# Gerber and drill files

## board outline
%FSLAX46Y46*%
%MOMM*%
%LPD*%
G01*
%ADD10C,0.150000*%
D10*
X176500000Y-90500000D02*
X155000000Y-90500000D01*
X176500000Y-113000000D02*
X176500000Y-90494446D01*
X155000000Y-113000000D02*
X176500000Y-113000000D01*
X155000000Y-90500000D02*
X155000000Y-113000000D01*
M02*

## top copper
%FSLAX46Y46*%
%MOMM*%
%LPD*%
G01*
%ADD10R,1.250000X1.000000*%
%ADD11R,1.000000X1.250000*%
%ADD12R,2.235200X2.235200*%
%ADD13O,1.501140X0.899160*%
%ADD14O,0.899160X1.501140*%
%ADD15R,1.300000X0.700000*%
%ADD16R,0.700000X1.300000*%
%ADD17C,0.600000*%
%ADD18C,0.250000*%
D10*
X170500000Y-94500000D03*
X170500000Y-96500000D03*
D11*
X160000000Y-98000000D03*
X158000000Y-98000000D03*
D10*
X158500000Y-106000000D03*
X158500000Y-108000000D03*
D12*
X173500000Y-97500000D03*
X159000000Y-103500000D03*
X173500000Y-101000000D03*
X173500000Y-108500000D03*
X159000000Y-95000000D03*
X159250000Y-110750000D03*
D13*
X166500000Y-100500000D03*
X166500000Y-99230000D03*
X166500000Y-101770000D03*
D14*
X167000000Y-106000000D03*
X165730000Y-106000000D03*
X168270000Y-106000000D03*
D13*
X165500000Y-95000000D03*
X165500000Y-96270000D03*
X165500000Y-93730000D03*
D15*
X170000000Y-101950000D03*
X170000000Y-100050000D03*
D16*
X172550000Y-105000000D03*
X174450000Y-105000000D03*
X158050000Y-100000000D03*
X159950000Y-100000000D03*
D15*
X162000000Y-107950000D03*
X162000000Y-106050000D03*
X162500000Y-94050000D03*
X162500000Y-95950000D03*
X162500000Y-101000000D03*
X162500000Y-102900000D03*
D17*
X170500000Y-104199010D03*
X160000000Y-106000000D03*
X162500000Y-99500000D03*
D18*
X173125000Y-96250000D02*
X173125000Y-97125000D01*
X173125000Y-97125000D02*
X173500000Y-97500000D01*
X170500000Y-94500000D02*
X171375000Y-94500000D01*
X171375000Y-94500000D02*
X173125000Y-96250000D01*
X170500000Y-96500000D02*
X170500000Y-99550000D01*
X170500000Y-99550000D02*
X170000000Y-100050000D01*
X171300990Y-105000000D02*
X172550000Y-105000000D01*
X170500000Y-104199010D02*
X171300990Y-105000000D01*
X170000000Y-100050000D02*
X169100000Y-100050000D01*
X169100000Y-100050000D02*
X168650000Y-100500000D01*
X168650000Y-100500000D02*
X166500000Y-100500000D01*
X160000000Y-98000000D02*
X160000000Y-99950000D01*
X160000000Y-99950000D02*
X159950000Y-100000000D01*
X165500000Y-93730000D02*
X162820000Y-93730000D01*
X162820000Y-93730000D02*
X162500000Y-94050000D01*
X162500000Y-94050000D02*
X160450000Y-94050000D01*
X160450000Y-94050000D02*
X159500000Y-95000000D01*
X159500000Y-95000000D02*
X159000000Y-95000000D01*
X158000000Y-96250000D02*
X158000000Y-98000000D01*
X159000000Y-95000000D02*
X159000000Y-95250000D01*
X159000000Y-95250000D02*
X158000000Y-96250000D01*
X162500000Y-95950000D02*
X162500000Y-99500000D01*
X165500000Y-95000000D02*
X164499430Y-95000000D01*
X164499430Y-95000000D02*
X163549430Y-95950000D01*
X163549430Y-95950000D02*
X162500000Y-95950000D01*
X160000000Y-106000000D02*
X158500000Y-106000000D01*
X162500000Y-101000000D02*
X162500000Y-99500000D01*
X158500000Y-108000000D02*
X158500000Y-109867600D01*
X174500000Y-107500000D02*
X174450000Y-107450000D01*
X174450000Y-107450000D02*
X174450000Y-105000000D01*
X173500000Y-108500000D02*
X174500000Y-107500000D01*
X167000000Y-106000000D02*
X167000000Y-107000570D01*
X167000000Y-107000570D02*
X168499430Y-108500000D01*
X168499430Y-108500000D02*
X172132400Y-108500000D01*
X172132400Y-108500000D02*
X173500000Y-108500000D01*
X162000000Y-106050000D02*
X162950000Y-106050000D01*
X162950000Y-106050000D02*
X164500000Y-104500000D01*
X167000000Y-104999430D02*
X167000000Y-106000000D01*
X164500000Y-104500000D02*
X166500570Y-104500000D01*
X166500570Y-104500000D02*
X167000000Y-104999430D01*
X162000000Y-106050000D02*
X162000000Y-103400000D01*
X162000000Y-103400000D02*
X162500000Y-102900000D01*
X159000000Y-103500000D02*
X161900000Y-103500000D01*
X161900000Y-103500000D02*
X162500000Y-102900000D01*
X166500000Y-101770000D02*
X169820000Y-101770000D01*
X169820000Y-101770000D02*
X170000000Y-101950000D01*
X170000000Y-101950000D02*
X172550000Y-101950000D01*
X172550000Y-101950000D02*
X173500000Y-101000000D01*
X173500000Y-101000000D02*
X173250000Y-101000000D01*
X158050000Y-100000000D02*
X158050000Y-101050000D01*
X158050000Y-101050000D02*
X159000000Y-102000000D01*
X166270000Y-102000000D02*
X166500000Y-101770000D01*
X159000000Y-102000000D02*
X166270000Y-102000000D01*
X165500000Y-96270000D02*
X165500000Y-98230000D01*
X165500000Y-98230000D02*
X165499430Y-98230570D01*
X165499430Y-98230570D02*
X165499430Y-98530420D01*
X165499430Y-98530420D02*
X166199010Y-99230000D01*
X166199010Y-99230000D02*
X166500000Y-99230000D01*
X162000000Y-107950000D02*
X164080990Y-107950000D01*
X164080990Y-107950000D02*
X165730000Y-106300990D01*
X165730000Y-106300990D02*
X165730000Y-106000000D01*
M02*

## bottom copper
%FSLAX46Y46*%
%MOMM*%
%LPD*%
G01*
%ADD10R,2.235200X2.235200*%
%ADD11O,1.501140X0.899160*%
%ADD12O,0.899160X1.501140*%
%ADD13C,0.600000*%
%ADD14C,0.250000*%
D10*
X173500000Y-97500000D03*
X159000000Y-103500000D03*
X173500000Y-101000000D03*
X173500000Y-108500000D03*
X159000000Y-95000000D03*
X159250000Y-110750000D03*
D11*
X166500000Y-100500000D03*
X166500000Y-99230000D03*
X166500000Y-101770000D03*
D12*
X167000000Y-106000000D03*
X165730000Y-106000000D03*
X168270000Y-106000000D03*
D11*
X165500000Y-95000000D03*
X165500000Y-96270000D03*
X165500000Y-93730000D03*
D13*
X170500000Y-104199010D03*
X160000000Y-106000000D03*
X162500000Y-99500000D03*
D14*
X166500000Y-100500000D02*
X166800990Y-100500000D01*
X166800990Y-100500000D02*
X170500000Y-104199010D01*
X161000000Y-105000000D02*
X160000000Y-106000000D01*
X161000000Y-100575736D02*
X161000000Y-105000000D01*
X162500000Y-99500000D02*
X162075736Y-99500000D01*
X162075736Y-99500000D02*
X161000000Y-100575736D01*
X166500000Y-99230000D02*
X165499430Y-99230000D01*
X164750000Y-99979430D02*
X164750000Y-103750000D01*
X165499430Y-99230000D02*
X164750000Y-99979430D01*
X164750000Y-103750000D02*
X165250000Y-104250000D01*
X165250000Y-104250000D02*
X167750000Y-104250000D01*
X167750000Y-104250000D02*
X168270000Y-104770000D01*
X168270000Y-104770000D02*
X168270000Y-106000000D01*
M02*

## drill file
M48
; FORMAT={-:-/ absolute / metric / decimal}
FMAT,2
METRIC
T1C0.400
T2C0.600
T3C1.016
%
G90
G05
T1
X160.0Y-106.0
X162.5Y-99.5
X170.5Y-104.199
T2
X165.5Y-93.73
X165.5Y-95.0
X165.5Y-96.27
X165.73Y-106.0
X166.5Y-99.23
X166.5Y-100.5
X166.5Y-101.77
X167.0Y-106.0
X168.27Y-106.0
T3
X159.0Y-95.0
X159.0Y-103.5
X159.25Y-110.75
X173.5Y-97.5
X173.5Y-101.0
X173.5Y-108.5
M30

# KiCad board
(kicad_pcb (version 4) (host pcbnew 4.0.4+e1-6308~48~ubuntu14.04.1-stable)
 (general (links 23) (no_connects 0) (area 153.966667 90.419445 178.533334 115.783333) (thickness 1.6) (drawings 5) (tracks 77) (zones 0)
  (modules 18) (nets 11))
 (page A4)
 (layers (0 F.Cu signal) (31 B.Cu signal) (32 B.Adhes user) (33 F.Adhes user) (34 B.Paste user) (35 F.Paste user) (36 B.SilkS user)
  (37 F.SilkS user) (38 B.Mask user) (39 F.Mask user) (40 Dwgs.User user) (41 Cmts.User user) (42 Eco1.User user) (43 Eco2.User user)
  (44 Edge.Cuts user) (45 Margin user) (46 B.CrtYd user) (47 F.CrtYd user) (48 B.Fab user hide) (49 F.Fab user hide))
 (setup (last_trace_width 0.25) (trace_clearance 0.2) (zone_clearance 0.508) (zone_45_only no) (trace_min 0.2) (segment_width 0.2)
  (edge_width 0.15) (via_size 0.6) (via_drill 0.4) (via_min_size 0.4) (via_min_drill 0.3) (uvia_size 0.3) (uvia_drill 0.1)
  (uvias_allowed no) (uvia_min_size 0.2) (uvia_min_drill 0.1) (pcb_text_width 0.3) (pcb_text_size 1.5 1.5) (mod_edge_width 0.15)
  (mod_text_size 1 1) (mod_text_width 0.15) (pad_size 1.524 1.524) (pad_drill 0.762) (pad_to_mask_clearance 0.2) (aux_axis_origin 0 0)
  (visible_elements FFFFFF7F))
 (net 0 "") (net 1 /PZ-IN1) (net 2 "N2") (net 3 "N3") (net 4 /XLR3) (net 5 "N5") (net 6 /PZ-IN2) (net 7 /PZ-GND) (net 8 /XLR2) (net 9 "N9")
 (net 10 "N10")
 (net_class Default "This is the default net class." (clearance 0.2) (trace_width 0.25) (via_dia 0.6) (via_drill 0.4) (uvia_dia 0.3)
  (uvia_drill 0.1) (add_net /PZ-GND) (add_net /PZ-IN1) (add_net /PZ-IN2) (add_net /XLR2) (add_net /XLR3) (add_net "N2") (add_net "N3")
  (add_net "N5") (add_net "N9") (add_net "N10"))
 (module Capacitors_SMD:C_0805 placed (layer F.Cu) (at 170.5 95.5 270)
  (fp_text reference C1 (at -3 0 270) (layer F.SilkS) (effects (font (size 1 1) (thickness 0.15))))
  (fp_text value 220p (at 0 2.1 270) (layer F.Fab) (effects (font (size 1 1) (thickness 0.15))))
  (pad 1 smd rect (at -1 0 270) (size 1 1.25) (layers F.Cu F.Paste F.Mask) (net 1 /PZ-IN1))
  (pad 2 smd rect (at 1 0 270) (size 1 1.25) (layers F.Cu F.Paste F.Mask) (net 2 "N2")))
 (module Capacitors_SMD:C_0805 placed (layer F.Cu) (at 159 98 180)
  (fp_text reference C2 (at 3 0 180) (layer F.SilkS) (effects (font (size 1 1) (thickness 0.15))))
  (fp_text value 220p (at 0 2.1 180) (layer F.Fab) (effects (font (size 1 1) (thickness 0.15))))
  (pad 1 smd rect (at -1 0 180) (size 1 1.25) (layers F.Cu F.Paste F.Mask) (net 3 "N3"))
  (pad 2 smd rect (at 1 0 180) (size 1 1.25) (layers F.Cu F.Paste F.Mask) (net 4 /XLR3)))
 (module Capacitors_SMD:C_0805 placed (layer F.Cu) (at 158.5 107 270)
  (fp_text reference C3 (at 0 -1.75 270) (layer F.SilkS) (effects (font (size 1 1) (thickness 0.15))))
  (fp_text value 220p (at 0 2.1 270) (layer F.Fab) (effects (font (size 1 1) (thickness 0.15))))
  (pad 1 smd rect (at -1 0 270) (size 1 1.25) (layers F.Cu F.Paste F.Mask) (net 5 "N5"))
  (pad 2 smd rect (at 1 0 270) (size 1 1.25) (layers F.Cu F.Paste F.Mask) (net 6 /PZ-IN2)))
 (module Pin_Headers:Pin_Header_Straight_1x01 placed (layer F.Cu) (at 173.5 97.5)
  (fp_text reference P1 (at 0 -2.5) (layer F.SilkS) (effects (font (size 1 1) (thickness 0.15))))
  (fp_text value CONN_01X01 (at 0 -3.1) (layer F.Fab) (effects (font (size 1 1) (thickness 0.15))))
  (pad 1 thru_hole rect (at 0 0) (size 2.2352 2.2352) (drill 1.016) (layers *.Cu *.Mask F.SilkS) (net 1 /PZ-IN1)))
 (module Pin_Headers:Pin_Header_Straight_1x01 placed (layer F.Cu) (at 159 103.5 90)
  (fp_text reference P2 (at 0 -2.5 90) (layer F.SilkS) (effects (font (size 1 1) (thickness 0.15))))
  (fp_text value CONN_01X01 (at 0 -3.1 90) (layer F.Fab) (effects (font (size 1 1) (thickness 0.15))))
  (pad 1 thru_hole rect (at 0 0 90) (size 2.2352 2.2352) (drill 1.016) (layers *.Cu *.Mask F.SilkS) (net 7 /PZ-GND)))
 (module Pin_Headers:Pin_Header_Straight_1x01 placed (layer F.Cu) (at 173.5 101)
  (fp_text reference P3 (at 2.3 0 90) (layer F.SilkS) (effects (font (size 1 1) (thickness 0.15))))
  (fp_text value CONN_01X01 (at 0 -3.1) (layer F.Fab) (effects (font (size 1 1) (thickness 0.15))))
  (pad 1 thru_hole rect (at 0 0) (size 2.2352 2.2352) (drill 1.016) (layers *.Cu *.Mask F.SilkS) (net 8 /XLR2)))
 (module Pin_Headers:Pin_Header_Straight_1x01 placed (layer F.Cu) (at 173.5 108.5)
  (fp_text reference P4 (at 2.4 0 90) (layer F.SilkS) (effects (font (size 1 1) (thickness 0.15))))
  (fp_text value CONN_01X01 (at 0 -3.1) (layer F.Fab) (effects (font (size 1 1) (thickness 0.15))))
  (pad 1 thru_hole rect (at 0 0) (size 2.2352 2.2352) (drill 1.016) (layers *.Cu *.Mask F.SilkS) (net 7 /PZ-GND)))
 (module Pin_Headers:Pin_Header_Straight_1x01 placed (layer F.Cu) (at 159 95)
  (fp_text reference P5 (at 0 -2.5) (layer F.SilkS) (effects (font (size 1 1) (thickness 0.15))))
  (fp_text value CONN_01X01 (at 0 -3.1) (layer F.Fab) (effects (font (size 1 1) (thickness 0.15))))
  (pad 1 thru_hole rect (at 0 0) (size 2.2352 2.2352) (drill 1.016) (layers *.Cu *.Mask F.SilkS) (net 4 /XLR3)))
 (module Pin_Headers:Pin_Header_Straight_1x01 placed (layer F.Cu) (at 159.25 110.75 90)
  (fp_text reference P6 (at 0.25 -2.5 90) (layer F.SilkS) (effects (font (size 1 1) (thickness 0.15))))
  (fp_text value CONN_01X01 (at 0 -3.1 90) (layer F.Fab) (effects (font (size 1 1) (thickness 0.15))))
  (pad 1 thru_hole rect (at 0 0 90) (size 2.2352 2.2352) (drill 1.016) (layers *.Cu *.Mask F.SilkS) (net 6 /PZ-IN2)))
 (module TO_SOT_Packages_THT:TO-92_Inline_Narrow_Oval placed (layer F.Cu) (at 166.5 101.77 90)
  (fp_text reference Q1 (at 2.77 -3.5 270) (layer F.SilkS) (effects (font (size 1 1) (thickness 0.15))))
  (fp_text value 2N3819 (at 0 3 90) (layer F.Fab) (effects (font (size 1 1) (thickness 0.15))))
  (pad 2 thru_hole oval (at 1.27 0 270) (size 0.89916 1.50114) (drill 0.6) (layers *.Cu *.Mask F.SilkS) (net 2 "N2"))
  (pad 3 thru_hole oval (at 2.54 0 270) (size 0.89916 1.50114) (drill 0.6) (layers *.Cu *.Mask F.SilkS) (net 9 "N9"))
  (pad 1 thru_hole oval (at 0 0 270) (size 0.89916 1.50114) (drill 0.6) (layers *.Cu *.Mask F.SilkS) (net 8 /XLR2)))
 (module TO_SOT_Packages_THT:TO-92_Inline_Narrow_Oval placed (layer F.Cu) (at 168.27 106 180)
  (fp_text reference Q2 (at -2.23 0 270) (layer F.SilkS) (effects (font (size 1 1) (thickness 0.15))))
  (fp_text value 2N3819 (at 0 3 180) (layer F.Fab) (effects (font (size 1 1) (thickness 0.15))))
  (pad 2 thru_hole oval (at 1.27 0) (size 0.89916 1.50114) (drill 0.6) (layers *.Cu *.Mask F.SilkS) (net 7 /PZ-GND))
  (pad 3 thru_hole oval (at 2.54 0) (size 0.89916 1.50114) (drill 0.6) (layers *.Cu *.Mask F.SilkS) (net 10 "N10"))
  (pad 1 thru_hole oval (at 0 0) (size 0.89916 1.50114) (drill 0.6) (layers *.Cu *.Mask F.SilkS) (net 9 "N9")))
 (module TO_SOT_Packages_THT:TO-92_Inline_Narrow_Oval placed (layer F.Cu) (at 165.5 93.73 270)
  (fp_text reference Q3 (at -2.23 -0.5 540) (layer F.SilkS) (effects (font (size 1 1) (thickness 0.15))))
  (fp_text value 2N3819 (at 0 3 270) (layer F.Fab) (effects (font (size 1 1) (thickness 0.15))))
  (pad 2 thru_hole oval (at 1.27 0 90) (size 0.89916 1.50114) (drill 0.6) (layers *.Cu *.Mask F.SilkS) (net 5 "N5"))
  (pad 3 thru_hole oval (at 2.54 0 90) (size 0.89916 1.50114) (drill 0.6) (layers *.Cu *.Mask F.SilkS) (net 9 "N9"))
  (pad 1 thru_hole oval (at 0 0 90) (size 0.89916 1.50114) (drill 0.6) (layers *.Cu *.Mask F.SilkS) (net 4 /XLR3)))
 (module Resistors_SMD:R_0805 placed (layer F.Cu) (at 170 101 90)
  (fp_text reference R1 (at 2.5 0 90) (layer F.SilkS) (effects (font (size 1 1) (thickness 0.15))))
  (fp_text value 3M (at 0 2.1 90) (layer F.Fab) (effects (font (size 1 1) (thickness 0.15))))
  (pad 1 smd rect (at -0.95 0 90) (size 0.7 1.3) (layers F.Cu F.Paste F.Mask) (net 8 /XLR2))
  (pad 2 smd rect (at 0.95 0 90) (size 0.7 1.3) (layers F.Cu F.Paste F.Mask) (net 2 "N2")))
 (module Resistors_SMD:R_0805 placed (layer F.Cu) (at 173.5 105)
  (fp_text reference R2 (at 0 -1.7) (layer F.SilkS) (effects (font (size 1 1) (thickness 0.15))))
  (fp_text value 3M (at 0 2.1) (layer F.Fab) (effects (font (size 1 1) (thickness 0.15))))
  (pad 1 smd rect (at -0.95 0) (size 0.7 1.3) (layers F.Cu F.Paste F.Mask) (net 2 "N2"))
  (pad 2 smd rect (at 0.95 0) (size 0.7 1.3) (layers F.Cu F.Paste F.Mask) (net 7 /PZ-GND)))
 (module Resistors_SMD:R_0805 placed (layer F.Cu) (at 159 100)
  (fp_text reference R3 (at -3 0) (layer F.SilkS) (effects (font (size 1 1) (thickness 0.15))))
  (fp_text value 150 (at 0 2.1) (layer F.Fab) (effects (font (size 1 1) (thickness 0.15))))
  (pad 1 smd rect (at -0.95 0) (size 0.7 1.3) (layers F.Cu F.Paste F.Mask) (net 8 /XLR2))
  (pad 2 smd rect (at 0.95 0) (size 0.7 1.3) (layers F.Cu F.Paste F.Mask) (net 3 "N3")))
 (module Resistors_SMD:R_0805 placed (layer F.Cu) (at 162 107 90)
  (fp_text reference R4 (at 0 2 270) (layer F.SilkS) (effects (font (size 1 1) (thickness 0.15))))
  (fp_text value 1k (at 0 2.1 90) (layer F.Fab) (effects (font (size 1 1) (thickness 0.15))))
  (pad 1 smd rect (at -0.95 0 90) (size 0.7 1.3) (layers F.Cu F.Paste F.Mask) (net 10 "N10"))
  (pad 2 smd rect (at 0.95 0 90) (size 0.7 1.3) (layers F.Cu F.Paste F.Mask) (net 7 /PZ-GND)))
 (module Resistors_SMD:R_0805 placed (layer F.Cu) (at 162.5 95 270)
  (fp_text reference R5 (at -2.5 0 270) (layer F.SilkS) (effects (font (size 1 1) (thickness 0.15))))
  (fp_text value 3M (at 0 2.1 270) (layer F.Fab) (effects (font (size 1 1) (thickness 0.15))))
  (pad 1 smd rect (at -0.95 0 270) (size 0.7 1.3) (layers F.Cu F.Paste F.Mask) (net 4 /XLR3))
  (pad 2 smd rect (at 0.95 0 270) (size 0.7 1.3) (layers F.Cu F.Paste F.Mask) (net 5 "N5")))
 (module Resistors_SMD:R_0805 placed (layer F.Cu) (at 162.5 101.95 270)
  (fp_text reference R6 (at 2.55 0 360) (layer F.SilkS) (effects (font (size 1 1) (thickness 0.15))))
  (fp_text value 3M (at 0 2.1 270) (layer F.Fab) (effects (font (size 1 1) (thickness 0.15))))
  (pad 1 smd rect (at -0.95 0 270) (size 0.7 1.3) (layers F.Cu F.Paste F.Mask) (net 5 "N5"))
  (pad 2 smd rect (at 0.95 0 270) (size 0.7 1.3) (layers F.Cu F.Paste F.Mask) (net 7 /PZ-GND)))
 (gr_line (start 176.5 90.5) (end 155 90.5) (layer Edge.Cuts) (width 0.15))
 (gr_line (start 176.5 113) (end 176.5 90.494446) (layer Edge.Cuts) (width 0.15))
 (gr_line (start 155 113) (end 176.5 113) (layer Edge.Cuts) (width 0.15))
 (gr_line (start 155 90.5) (end 155 113) (layer Edge.Cuts) (width 0.15))
 (segment (start 173.125 96.25) (end 173.125 97.125) (width 0.25) (layer F.Cu) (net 1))
 (segment (start 173.125 97.125) (end 173.5 97.5) (width 0.25) (layer F.Cu) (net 1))
 (segment (start 170.5 94.5) (end 171.375 94.5) (width 0.25) (layer F.Cu) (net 1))
 (segment (start 171.375 94.5) (end 173.125 96.25) (width 0.25) (layer F.Cu) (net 1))
 (segment (start 170.5 96.5) (end 170.5 99.55) (width 0.25) (layer F.Cu) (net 2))
 (segment (start 170.5 99.55) (end 170 100.05) (width 0.25) (layer F.Cu) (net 2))
 (segment (start 171.30099 105) (end 172.55 105) (width 0.25) (layer F.Cu) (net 2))
 (segment (start 170.5 104.19901) (end 171.30099 105) (width 0.25) (layer F.Cu) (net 2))
 (via (at 170.5 104.19901) (size 0.6) (drill 0.4) (layers F.Cu B.Cu) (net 2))
 (segment (start 166.5 100.5) (end 166.80099 100.5) (width 0.25) (layer B.Cu) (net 2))
 (segment (start 166.80099 100.5) (end 170.5 104.19901) (width 0.25) (layer B.Cu) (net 2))
 (segment (start 170 100.05) (end 169.1 100.05) (width 0.25) (layer F.Cu) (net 2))
 (segment (start 169.1 100.05) (end 168.65 100.5) (width 0.25) (layer F.Cu) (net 2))
 (segment (start 168.65 100.5) (end 166.5 100.5) (width 0.25) (layer F.Cu) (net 2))
 (segment (start 160 98) (end 160 99.95) (width 0.25) (layer F.Cu) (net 3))
 (segment (start 160 99.95) (end 159.95 100) (width 0.25) (layer F.Cu) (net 3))
 (segment (start 165.5 93.73) (end 162.82 93.73) (width 0.25) (layer F.Cu) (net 4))
 (segment (start 162.82 93.73) (end 162.5 94.05) (width 0.25) (layer F.Cu) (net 4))
 (segment (start 162.5 94.05) (end 160.45 94.05) (width 0.25) (layer F.Cu) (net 4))
 (segment (start 160.45 94.05) (end 159.5 95) (width 0.25) (layer F.Cu) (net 4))
 (segment (start 159.5 95) (end 159 95) (width 0.25) (layer F.Cu) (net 4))
 (segment (start 158 96.25) (end 158 98) (width 0.25) (layer F.Cu) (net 4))
 (segment (start 159 95) (end 159 95.25) (width 0.25) (layer F.Cu) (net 4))
 (segment (start 159 95.25) (end 158 96.25) (width 0.25) (layer F.Cu) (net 4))
 (segment (start 162.5 95.95) (end 162.5 99.5) (width 0.25) (layer F.Cu) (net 5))
 (segment (start 165.5 95) (end 164.49943 95) (width 0.25) (layer F.Cu) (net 5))
 (segment (start 164.49943 95) (end 163.54943 95.95) (width 0.25) (layer F.Cu) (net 5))
 (segment (start 163.54943 95.95) (end 162.5 95.95) (width 0.25) (layer F.Cu) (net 5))
 (segment (start 160 106) (end 158.5 106) (width 0.25) (layer F.Cu) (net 5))
 (via (at 160 106) (size 0.6) (drill 0.4) (layers F.Cu B.Cu) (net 5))
 (segment (start 161 105) (end 160 106) (width 0.25) (layer B.Cu) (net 5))
 (segment (start 161 100.575736) (end 161 105) (width 0.25) (layer B.Cu) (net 5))
 (segment (start 162.5 99.5) (end 162.075736 99.5) (width 0.25) (layer B.Cu) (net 5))
 (segment (start 162.075736 99.5) (end 161 100.575736) (width 0.25) (layer B.Cu) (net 5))
 (segment (start 162.5 101) (end 162.5 99.5) (width 0.25) (layer F.Cu) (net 5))
 (via (at 162.5 99.5) (size 0.6) (drill 0.4) (layers F.Cu B.Cu) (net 5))
 (segment (start 158.5 108) (end 158.5 109.8676) (width 0.25) (layer F.Cu) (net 6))
 (segment (start 174.5 107.5) (end 174.45 107.45) (width 0.25) (layer F.Cu) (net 7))
 (segment (start 174.45 107.45) (end 174.45 105) (width 0.25) (layer F.Cu) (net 7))
 (segment (start 173.5 108.5) (end 174.5 107.5) (width 0.25) (layer F.Cu) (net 7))
 (segment (start 167 106) (end 167 107.00057) (width 0.25) (layer F.Cu) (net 7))
 (segment (start 167 107.00057) (end 168.49943 108.5) (width 0.25) (layer F.Cu) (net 7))
 (segment (start 168.49943 108.5) (end 172.1324 108.5) (width 0.25) (layer F.Cu) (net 7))
 (segment (start 172.1324 108.5) (end 173.5 108.5) (width 0.25) (layer F.Cu) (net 7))
 (segment (start 162 106.05) (end 162.95 106.05) (width 0.25) (layer F.Cu) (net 7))
 (segment (start 162.95 106.05) (end 164.5 104.5) (width 0.25) (layer F.Cu) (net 7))
 (segment (start 167 104.99943) (end 167 106) (width 0.25) (layer F.Cu) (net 7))
 (segment (start 164.5 104.5) (end 166.50057 104.5) (width 0.25) (layer F.Cu) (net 7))
 (segment (start 166.50057 104.5) (end 167 104.99943) (width 0.25) (layer F.Cu) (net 7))
 (segment (start 162 106.05) (end 162 103.4) (width 0.25) (layer F.Cu) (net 7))
 (segment (start 162 103.4) (end 162.5 102.9) (width 0.25) (layer F.Cu) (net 7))
 (segment (start 159 103.5) (end 161.9 103.5) (width 0.25) (layer F.Cu) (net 7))
 (segment (start 161.9 103.5) (end 162.5 102.9) (width 0.25) (layer F.Cu) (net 7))
 (segment (start 166.5 101.77) (end 169.82 101.77) (width 0.25) (layer F.Cu) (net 8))
 (segment (start 169.82 101.77) (end 170 101.95) (width 0.25) (layer F.Cu) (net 8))
 (segment (start 170 101.95) (end 172.55 101.95) (width 0.25) (layer F.Cu) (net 8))
 (segment (start 172.55 101.95) (end 173.5 101) (width 0.25) (layer F.Cu) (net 8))
 (segment (start 173.5 101) (end 173.25 101) (width 0.25) (layer F.Cu) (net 8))
 (segment (start 158.05 100) (end 158.05 101.05) (width 0.25) (layer F.Cu) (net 8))
 (segment (start 158.05 101.05) (end 159 102) (width 0.25) (layer F.Cu) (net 8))
 (segment (start 166.27 102) (end 166.5 101.77) (width 0.25) (layer F.Cu) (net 8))
 (segment (start 159 102) (end 166.27 102) (width 0.25) (layer F.Cu) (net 8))
 (segment (start 166.5 99.23) (end 165.49943 99.23) (width 0.25) (layer B.Cu) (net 9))
 (segment (start 164.75 99.97943) (end 164.75 103.75) (width 0.25) (layer B.Cu) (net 9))
 (segment (start 165.49943 99.23) (end 164.75 99.97943) (width 0.25) (layer B.Cu) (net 9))
 (segment (start 164.75 103.75) (end 165.25 104.25) (width 0.25) (layer B.Cu) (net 9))
 (segment (start 165.25 104.25) (end 167.75 104.25) (width 0.25) (layer B.Cu) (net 9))
 (segment (start 167.75 104.25) (end 168.27 104.77) (width 0.25) (layer B.Cu) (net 9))
 (segment (start 168.27 104.77) (end 168.27 106) (width 0.25) (layer B.Cu) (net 9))
 (segment (start 165.5 96.27) (end 165.5 98.23) (width 0.25) (layer F.Cu) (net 9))
 (segment (start 165.5 98.23) (end 165.49943 98.23057) (width 0.25) (layer F.Cu) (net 9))
 (segment (start 165.49943 98.23057) (end 165.49943 98.53042) (width 0.25) (layer F.Cu) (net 9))
 (segment (start 165.49943 98.53042) (end 166.19901 99.23) (width 0.25) (layer F.Cu) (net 9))
 (segment (start 166.19901 99.23) (end 166.5 99.23) (width 0.25) (layer F.Cu) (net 9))
 (segment (start 162 107.95) (end 164.08099 107.95) (width 0.25) (layer F.Cu) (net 10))
 (segment (start 164.08099 107.95) (end 165.73 106.30099) (width 0.25) (layer F.Cu) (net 10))
 (segment (start 165.73 106.30099) (end 165.73 106) (width 0.25) (layer F.Cu) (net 10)))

